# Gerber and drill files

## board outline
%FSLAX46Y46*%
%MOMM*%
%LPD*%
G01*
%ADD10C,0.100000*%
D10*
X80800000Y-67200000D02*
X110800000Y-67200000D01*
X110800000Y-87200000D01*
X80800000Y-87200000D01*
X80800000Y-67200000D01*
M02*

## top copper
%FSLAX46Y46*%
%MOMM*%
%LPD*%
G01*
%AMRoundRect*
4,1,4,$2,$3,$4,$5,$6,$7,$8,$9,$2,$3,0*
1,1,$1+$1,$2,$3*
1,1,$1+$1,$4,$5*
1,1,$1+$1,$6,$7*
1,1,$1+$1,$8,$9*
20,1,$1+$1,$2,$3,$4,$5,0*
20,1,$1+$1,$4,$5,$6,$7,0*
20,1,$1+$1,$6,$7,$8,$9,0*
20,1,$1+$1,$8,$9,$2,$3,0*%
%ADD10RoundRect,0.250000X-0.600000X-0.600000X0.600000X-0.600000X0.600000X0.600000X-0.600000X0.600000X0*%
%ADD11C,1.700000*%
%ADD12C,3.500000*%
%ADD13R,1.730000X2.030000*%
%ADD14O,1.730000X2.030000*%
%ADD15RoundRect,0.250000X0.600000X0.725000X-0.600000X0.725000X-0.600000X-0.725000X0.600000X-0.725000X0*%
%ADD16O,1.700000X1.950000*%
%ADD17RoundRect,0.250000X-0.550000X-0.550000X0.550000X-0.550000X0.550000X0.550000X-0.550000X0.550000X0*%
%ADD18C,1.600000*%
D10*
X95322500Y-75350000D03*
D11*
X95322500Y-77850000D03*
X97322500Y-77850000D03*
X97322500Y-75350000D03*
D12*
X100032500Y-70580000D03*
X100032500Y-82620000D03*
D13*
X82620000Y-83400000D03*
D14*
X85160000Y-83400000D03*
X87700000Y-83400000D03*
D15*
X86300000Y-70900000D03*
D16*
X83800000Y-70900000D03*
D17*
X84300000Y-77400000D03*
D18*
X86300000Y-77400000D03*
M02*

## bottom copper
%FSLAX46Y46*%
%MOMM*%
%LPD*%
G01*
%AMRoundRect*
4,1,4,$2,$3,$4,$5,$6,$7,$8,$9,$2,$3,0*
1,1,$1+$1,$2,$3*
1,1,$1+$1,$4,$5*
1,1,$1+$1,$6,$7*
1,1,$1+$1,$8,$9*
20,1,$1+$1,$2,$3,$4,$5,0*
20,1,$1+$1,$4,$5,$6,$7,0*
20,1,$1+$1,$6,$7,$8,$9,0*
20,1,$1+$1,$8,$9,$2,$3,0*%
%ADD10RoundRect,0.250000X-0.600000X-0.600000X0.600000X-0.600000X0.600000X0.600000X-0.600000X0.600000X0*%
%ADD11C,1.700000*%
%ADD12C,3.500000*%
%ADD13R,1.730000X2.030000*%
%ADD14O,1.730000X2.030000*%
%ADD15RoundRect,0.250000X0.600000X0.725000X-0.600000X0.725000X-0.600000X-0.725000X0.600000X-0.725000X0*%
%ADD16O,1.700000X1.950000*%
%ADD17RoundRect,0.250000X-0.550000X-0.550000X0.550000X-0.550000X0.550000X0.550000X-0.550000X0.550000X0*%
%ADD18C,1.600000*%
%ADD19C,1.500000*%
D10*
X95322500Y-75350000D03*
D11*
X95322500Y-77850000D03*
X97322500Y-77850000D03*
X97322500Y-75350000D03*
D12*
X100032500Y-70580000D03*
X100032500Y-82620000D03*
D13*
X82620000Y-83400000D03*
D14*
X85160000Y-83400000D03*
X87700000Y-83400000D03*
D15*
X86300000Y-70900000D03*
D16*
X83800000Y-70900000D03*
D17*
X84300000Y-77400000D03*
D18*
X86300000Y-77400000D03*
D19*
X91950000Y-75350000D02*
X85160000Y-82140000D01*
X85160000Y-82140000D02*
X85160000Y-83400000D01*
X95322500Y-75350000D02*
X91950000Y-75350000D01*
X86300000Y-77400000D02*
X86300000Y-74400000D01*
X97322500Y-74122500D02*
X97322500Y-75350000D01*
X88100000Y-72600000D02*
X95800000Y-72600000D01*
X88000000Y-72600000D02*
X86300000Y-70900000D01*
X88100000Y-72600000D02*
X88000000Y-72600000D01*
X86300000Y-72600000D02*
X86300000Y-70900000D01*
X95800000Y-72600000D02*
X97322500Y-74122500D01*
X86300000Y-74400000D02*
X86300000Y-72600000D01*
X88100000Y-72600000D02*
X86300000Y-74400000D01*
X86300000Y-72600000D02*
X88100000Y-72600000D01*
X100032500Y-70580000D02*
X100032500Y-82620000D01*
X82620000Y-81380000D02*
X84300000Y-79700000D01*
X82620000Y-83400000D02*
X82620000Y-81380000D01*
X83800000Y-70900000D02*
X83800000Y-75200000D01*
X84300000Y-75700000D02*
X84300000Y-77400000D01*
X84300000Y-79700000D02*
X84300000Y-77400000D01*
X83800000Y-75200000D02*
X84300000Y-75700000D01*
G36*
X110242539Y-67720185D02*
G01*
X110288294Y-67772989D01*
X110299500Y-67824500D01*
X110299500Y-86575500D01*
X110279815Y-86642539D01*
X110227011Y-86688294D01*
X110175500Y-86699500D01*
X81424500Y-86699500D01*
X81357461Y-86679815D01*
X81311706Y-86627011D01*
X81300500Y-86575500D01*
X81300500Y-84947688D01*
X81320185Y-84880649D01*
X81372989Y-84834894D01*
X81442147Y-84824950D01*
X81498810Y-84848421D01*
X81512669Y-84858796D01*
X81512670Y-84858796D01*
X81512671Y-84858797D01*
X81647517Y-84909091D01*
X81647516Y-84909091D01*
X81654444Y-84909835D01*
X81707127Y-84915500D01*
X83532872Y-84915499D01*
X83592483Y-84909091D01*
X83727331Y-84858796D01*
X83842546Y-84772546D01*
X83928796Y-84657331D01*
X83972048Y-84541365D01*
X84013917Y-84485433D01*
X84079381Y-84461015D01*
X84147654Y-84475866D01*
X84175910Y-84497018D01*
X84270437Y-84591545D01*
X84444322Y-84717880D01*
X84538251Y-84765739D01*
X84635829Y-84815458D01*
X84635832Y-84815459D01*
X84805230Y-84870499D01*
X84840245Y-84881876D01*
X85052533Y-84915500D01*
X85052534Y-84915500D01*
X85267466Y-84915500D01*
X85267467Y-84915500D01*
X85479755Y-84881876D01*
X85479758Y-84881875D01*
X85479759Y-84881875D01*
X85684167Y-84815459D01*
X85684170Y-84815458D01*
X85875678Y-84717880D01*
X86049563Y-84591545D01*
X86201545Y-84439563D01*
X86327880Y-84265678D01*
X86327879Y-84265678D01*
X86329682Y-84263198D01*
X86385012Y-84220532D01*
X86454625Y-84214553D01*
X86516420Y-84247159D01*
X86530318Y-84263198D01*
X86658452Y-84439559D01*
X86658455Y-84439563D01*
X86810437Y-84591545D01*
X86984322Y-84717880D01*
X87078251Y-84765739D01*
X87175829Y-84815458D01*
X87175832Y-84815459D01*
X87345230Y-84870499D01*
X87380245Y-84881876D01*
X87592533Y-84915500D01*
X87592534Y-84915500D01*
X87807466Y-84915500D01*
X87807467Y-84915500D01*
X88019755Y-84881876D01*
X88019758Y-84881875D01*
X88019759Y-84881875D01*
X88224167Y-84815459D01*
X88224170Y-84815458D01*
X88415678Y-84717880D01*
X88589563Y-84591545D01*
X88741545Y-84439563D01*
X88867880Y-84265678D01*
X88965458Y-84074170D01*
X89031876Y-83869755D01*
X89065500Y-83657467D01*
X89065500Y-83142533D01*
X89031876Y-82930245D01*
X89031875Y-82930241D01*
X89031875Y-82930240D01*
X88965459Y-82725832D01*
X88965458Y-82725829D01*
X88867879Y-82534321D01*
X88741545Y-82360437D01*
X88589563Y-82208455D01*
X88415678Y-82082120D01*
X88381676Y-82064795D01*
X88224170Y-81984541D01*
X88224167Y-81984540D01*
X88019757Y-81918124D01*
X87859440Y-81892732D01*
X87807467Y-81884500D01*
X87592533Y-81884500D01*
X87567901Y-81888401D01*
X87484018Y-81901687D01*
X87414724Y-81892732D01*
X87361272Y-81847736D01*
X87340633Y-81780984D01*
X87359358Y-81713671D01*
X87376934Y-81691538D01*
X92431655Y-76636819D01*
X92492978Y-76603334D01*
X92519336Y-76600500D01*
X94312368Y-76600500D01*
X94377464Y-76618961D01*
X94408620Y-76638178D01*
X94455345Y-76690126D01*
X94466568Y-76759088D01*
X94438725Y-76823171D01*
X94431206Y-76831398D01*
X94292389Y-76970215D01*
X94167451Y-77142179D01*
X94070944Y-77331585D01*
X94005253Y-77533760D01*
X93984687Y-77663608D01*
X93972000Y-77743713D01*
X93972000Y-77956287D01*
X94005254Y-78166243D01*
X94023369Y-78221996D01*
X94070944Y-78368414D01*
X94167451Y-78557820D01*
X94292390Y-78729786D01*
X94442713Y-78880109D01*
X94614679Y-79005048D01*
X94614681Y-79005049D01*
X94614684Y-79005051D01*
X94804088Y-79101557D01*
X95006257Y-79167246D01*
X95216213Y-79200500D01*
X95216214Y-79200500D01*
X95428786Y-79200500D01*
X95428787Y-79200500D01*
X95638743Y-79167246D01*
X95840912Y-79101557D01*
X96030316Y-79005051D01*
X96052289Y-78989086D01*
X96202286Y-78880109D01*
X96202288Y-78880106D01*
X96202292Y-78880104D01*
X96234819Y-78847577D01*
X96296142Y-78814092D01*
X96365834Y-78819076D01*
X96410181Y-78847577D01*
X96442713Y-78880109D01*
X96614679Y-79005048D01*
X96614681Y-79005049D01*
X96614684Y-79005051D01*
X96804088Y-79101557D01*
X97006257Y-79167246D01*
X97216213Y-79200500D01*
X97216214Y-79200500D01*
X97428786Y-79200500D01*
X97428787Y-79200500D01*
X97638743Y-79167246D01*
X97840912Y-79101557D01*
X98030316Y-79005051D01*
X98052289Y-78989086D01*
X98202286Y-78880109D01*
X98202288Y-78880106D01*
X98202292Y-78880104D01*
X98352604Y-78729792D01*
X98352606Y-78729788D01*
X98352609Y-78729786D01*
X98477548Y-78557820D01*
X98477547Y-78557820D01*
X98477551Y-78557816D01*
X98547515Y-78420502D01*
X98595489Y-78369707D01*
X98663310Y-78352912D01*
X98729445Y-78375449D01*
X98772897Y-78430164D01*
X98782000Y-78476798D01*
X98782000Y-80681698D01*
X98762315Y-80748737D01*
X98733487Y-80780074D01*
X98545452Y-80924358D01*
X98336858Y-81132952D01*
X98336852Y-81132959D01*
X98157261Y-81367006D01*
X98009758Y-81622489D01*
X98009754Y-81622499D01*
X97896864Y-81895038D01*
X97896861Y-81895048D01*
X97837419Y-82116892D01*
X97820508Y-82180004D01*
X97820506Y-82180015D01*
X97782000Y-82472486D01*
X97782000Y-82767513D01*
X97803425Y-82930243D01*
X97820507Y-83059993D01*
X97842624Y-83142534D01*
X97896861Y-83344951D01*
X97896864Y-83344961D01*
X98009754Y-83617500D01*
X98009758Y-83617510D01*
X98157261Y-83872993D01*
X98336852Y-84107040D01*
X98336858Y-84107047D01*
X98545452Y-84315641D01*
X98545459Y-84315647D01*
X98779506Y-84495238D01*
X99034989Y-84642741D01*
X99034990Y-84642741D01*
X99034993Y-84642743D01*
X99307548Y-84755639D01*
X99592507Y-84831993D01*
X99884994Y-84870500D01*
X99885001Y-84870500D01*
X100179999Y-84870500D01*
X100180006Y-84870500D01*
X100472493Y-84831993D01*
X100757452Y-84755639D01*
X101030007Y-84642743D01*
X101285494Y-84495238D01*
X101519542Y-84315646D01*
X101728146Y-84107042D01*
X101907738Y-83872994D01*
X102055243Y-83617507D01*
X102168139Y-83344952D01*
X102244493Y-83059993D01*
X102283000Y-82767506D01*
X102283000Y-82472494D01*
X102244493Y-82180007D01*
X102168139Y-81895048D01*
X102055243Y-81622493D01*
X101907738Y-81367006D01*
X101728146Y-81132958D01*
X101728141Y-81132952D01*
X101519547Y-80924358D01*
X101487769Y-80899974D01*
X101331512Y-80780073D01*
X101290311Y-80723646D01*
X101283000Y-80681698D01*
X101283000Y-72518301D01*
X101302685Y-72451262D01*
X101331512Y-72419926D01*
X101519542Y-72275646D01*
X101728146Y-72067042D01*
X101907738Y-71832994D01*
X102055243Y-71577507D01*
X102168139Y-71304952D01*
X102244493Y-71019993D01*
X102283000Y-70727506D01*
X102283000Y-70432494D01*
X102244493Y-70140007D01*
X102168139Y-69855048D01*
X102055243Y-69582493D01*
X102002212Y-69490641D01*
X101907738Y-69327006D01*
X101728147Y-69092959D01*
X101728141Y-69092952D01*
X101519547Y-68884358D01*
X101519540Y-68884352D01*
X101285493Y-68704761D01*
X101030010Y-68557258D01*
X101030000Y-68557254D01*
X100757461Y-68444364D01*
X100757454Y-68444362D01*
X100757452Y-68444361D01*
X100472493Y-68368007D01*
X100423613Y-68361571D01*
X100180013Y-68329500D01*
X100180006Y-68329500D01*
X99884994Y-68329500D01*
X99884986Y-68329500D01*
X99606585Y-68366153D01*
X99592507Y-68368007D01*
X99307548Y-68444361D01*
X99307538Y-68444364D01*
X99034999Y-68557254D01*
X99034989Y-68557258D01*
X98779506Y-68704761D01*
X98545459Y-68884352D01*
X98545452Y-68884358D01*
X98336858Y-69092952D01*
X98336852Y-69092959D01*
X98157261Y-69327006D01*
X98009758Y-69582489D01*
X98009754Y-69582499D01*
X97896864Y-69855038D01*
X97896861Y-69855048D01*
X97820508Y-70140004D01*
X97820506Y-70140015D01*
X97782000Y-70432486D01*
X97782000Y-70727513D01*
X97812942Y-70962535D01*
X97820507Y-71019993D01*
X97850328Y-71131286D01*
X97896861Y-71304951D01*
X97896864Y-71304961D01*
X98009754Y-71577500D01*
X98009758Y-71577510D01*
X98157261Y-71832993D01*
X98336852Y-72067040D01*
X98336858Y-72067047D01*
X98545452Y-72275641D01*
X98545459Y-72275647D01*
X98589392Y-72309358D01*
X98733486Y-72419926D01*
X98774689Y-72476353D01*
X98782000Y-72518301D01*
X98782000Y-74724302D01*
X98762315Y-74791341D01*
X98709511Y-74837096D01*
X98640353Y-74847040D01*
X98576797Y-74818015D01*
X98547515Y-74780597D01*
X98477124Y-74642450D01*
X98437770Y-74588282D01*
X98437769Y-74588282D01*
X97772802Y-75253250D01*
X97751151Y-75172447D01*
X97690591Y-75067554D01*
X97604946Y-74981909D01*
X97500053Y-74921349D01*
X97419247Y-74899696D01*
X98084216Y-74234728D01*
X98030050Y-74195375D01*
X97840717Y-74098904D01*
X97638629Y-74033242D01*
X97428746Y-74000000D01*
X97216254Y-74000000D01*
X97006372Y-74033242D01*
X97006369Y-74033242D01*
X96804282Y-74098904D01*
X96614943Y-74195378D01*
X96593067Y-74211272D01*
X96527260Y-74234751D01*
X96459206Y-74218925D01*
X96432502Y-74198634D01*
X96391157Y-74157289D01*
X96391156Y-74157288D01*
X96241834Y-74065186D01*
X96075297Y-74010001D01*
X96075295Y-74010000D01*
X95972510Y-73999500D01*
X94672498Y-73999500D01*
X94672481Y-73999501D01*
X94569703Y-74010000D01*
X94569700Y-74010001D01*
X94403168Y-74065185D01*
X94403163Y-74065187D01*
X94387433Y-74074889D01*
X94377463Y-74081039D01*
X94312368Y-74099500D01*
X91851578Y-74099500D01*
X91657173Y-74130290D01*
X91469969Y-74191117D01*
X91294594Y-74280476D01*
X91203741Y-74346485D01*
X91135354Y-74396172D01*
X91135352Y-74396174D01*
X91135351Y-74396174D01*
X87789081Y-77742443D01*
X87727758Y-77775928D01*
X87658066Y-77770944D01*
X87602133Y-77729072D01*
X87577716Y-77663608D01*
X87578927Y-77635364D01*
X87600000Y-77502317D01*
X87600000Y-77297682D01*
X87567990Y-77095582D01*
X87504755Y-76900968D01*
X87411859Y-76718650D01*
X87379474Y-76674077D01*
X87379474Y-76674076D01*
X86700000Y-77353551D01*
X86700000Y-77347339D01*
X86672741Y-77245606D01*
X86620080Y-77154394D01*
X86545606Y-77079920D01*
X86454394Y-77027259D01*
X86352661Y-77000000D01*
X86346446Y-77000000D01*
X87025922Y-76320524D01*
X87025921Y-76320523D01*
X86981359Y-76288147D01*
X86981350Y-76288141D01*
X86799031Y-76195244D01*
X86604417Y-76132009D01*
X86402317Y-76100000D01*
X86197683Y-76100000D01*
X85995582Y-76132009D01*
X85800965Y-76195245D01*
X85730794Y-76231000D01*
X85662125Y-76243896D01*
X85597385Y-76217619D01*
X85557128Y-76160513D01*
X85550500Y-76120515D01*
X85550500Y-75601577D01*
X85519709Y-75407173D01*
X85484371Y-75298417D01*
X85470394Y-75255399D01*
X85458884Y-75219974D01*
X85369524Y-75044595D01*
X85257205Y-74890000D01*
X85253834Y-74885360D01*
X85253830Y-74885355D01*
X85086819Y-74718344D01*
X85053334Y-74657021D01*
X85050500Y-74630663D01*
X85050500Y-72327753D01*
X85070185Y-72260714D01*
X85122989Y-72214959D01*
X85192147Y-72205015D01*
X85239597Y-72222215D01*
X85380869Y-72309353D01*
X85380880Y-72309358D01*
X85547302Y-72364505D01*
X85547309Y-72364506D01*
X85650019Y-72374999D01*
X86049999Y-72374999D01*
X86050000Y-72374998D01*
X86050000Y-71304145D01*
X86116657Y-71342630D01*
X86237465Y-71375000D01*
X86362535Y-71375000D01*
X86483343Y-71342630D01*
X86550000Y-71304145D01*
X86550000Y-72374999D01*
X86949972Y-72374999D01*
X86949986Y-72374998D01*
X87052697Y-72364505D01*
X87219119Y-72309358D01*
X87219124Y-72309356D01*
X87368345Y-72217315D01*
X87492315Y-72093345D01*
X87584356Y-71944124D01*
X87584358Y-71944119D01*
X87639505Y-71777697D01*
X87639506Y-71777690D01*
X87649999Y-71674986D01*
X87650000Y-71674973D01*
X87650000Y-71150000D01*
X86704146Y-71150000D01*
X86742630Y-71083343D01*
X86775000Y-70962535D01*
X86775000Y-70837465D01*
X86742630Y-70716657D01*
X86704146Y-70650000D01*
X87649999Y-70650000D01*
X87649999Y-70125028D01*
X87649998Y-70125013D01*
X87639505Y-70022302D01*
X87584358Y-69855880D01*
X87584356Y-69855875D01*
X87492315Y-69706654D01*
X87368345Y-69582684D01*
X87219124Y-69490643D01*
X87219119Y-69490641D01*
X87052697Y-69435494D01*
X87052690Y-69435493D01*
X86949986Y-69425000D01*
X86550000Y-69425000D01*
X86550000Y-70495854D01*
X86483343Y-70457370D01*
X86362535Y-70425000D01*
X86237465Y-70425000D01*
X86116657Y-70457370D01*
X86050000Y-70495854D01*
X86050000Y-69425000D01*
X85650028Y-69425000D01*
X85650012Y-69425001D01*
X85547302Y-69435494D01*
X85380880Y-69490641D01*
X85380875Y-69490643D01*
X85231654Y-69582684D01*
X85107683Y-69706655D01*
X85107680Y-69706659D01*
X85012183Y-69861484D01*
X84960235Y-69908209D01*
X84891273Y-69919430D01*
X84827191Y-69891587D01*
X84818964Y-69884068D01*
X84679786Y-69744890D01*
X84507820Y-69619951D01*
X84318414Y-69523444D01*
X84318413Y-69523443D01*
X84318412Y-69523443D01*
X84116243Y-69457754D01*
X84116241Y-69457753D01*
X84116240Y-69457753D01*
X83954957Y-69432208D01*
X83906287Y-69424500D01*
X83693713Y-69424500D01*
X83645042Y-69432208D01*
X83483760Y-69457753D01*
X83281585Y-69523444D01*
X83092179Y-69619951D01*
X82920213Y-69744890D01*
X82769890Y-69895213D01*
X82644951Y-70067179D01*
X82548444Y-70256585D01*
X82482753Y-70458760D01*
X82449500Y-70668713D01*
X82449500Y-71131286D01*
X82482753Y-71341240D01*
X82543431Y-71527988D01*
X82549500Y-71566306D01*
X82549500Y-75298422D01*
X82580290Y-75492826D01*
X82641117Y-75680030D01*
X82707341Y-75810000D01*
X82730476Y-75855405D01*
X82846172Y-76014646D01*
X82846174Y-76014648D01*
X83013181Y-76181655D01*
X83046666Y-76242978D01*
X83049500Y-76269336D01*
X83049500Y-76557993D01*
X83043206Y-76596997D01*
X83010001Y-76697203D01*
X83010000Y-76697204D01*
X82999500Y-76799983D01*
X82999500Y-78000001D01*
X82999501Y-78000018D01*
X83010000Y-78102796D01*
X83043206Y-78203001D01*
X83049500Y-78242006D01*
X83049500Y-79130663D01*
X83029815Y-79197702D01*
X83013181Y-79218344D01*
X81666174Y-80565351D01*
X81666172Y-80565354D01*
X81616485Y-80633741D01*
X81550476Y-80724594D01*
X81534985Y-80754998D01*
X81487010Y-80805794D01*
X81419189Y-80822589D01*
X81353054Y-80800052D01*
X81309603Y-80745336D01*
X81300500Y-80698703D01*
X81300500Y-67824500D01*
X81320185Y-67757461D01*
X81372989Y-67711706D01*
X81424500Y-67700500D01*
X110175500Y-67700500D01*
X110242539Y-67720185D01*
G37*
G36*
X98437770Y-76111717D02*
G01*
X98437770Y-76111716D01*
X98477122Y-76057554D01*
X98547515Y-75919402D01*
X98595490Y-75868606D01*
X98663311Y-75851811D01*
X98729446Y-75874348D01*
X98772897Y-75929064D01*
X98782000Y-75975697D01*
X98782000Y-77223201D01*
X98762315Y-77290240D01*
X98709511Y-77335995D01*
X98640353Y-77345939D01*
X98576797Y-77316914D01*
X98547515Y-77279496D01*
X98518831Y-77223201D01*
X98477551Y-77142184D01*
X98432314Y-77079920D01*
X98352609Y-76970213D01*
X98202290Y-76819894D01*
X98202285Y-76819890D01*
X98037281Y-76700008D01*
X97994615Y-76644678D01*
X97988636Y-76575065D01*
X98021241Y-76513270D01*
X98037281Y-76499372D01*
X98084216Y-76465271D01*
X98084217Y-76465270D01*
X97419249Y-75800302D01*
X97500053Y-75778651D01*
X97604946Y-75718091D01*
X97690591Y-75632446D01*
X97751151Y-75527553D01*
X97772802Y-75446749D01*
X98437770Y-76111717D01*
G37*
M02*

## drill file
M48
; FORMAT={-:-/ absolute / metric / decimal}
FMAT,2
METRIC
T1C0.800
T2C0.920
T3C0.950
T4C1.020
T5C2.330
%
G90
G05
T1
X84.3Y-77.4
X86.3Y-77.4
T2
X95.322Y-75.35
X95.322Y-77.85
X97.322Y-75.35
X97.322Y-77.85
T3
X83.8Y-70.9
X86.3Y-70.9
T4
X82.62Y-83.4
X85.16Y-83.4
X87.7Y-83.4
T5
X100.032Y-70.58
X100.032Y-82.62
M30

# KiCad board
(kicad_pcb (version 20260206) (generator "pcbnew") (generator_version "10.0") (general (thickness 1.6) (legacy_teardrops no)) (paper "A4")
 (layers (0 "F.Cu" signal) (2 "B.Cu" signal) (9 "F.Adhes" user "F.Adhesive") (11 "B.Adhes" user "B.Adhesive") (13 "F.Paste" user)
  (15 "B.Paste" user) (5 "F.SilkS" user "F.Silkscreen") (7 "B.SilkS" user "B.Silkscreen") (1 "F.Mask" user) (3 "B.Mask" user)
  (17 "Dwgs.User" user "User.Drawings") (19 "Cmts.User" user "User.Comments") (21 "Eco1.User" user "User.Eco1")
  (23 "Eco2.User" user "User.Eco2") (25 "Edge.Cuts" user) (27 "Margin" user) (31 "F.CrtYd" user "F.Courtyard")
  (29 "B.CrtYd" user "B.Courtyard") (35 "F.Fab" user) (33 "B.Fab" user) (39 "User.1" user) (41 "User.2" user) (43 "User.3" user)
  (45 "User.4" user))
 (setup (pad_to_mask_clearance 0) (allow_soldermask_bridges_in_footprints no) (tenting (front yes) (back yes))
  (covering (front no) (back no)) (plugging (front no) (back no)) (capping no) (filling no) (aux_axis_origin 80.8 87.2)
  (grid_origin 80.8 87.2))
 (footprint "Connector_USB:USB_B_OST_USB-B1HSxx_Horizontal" (layer "F.Cu") (at 95.3225 75.35)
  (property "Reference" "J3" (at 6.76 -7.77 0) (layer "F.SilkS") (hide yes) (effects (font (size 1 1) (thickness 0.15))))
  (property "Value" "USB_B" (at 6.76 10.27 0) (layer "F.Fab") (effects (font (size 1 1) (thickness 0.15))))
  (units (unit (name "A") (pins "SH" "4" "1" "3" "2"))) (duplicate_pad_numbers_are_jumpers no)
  (pad "1" thru_hole roundrect (at 0 0) (size 1.7 1.7) (drill 0.92) (layers "*.Cu" "*.Mask") (remove_unused_layers no)
   (roundrect_rratio 0.1470588235) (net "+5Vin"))
  (pad "2" thru_hole circle (at 0 2.5) (size 1.7 1.7) (drill 0.92) (layers "*.Cu" "*.Mask") (remove_unused_layers no)
   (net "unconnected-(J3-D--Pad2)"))
  (pad "3" thru_hole circle (at 2 2.5) (size 1.7 1.7) (drill 0.92) (layers "*.Cu" "*.Mask") (remove_unused_layers no)
   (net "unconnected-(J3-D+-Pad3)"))
  (pad "4" thru_hole circle (at 2 0) (size 1.7 1.7) (drill 0.92) (layers "*.Cu" "*.Mask") (remove_unused_layers no) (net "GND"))
  (pad "SH" thru_hole circle (at 4.71 -4.77) (size 3.5 3.5) (drill 2.33) (layers "*.Cu" "*.Mask") (remove_unused_layers no)
   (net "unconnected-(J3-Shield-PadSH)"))
  (pad "SH" thru_hole circle (at 4.71 7.27) (size 3.5 3.5) (drill 2.33) (layers "*.Cu" "*.Mask") (remove_unused_layers no)
   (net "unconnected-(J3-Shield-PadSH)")))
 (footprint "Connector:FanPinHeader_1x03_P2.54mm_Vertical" (layer "F.Cu") (at 82.62 83.4)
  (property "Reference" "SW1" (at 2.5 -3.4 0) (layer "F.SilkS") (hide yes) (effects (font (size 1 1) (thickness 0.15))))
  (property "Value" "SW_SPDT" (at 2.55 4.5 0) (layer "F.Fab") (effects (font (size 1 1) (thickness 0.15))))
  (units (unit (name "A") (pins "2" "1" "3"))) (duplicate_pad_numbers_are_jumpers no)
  (pad "1" thru_hole rect (at 0 0 90) (size 2.03 1.73) (drill 1.02) (layers "*.Cu" "*.Mask") (remove_unused_layers no) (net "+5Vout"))
  (pad "2" thru_hole oval (at 2.54 0 90) (size 2.03 1.73) (drill 1.02) (layers "*.Cu" "*.Mask") (remove_unused_layers no) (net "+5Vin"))
  (pad "3" thru_hole oval (at 5.08 0 90) (size 2.03 1.73) (drill 1.02) (layers "*.Cu" "*.Mask") (remove_unused_layers no)
   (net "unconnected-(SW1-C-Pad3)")))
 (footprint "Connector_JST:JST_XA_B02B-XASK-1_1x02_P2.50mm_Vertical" (layer "F.Cu") (at 86.3 70.9 180)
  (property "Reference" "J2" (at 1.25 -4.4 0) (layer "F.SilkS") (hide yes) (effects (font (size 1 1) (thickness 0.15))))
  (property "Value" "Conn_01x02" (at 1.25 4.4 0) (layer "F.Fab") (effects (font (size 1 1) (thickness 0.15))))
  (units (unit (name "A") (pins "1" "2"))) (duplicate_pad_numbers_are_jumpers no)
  (pad "1" thru_hole roundrect (at 0 0 180) (size 1.7 1.95) (drill 0.95) (layers "*.Cu" "*.Mask") (remove_unused_layers no)
   (roundrect_rratio 0.147059) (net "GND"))
  (pad "2" thru_hole oval (at 2.5 0 180) (size 1.7 1.95) (drill 0.95) (layers "*.Cu" "*.Mask") (remove_unused_layers no) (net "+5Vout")))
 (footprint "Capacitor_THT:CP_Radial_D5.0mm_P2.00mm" (layer "F.Cu") (at 84.3 77.4)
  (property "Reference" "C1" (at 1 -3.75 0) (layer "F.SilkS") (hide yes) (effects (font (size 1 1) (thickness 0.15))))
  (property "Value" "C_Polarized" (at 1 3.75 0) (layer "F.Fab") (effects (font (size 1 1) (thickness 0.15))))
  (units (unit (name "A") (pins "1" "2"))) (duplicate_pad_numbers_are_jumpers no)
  (pad "1" thru_hole roundrect (at 0 0) (size 1.6 1.6) (drill 0.8) (layers "*.Cu" "*.Mask") (remove_unused_layers no)
   (roundrect_rratio 0.15625) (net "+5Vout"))
  (pad "2" thru_hole circle (at 2 0) (size 1.6 1.6) (drill 0.8) (layers "*.Cu" "*.Mask") (remove_unused_layers no) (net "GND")))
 (gr_rect (start 80.8 67.2) (end 110.8 87.2) (stroke (width 0.1) (type solid)) (fill no) (layer "Edge.Cuts"))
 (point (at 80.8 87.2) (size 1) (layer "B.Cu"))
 (segment (start 91.95 75.35) (end 85.16 82.14) (width 1.5) (layer "B.Cu") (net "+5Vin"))
 (segment (start 85.16 82.14) (end 85.16 83.4) (width 1.5) (layer "B.Cu") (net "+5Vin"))
 (segment (start 95.3225 75.35) (end 91.95 75.35) (width 1.5) (layer "B.Cu") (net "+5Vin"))
 (segment (start 86.3 77.4) (end 86.3 74.4) (width 1.5) (layer "B.Cu") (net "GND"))
 (segment (start 97.3225 74.1225) (end 97.3225 75.35) (width 1.5) (layer "B.Cu") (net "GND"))
 (segment (start 88.1 72.6) (end 95.8 72.6) (width 1.5) (layer "B.Cu") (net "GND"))
 (segment (start 88 72.6) (end 86.3 70.9) (width 1.5) (layer "B.Cu") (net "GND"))
 (segment (start 88.1 72.6) (end 88 72.6) (width 1.5) (layer "B.Cu") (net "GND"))
 (segment (start 86.3 72.6) (end 86.3 70.9) (width 1.5) (layer "B.Cu") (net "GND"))
 (segment (start 95.8 72.6) (end 97.3225 74.1225) (width 1.5) (layer "B.Cu") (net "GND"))
 (segment (start 86.3 74.4) (end 86.3 72.6) (width 1.5) (layer "B.Cu") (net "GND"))
 (segment (start 88.1 72.6) (end 86.3 74.4) (width 1.5) (layer "B.Cu") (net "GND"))
 (segment (start 86.3 72.6) (end 88.1 72.6) (width 1.5) (layer "B.Cu") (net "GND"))
 (segment (start 100.0325 70.58) (end 100.0325 82.62) (width 1.5) (layer "B.Cu") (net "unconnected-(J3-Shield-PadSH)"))
 (segment (start 82.62 81.38) (end 84.3 79.7) (width 1.5) (layer "B.Cu") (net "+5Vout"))
 (segment (start 82.62 83.4) (end 82.62 81.38) (width 1.5) (layer "B.Cu") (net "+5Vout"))
 (segment (start 83.8 70.9) (end 83.8 75.2) (width 1.5) (layer "B.Cu") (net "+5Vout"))
 (segment (start 84.3 75.7) (end 84.3 77.4) (width 1.5) (layer "B.Cu") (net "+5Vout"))
 (segment (start 84.3 79.7) (end 84.3 77.4) (width 1.5) (layer "B.Cu") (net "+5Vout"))
 (segment (start 83.8 75.2) (end 84.3 75.7) (width 1.5) (layer "B.Cu") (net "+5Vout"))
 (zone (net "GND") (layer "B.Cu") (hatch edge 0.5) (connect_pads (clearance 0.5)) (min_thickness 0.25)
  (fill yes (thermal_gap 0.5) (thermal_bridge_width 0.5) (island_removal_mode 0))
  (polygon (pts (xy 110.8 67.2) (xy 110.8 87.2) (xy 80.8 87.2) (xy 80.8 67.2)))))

